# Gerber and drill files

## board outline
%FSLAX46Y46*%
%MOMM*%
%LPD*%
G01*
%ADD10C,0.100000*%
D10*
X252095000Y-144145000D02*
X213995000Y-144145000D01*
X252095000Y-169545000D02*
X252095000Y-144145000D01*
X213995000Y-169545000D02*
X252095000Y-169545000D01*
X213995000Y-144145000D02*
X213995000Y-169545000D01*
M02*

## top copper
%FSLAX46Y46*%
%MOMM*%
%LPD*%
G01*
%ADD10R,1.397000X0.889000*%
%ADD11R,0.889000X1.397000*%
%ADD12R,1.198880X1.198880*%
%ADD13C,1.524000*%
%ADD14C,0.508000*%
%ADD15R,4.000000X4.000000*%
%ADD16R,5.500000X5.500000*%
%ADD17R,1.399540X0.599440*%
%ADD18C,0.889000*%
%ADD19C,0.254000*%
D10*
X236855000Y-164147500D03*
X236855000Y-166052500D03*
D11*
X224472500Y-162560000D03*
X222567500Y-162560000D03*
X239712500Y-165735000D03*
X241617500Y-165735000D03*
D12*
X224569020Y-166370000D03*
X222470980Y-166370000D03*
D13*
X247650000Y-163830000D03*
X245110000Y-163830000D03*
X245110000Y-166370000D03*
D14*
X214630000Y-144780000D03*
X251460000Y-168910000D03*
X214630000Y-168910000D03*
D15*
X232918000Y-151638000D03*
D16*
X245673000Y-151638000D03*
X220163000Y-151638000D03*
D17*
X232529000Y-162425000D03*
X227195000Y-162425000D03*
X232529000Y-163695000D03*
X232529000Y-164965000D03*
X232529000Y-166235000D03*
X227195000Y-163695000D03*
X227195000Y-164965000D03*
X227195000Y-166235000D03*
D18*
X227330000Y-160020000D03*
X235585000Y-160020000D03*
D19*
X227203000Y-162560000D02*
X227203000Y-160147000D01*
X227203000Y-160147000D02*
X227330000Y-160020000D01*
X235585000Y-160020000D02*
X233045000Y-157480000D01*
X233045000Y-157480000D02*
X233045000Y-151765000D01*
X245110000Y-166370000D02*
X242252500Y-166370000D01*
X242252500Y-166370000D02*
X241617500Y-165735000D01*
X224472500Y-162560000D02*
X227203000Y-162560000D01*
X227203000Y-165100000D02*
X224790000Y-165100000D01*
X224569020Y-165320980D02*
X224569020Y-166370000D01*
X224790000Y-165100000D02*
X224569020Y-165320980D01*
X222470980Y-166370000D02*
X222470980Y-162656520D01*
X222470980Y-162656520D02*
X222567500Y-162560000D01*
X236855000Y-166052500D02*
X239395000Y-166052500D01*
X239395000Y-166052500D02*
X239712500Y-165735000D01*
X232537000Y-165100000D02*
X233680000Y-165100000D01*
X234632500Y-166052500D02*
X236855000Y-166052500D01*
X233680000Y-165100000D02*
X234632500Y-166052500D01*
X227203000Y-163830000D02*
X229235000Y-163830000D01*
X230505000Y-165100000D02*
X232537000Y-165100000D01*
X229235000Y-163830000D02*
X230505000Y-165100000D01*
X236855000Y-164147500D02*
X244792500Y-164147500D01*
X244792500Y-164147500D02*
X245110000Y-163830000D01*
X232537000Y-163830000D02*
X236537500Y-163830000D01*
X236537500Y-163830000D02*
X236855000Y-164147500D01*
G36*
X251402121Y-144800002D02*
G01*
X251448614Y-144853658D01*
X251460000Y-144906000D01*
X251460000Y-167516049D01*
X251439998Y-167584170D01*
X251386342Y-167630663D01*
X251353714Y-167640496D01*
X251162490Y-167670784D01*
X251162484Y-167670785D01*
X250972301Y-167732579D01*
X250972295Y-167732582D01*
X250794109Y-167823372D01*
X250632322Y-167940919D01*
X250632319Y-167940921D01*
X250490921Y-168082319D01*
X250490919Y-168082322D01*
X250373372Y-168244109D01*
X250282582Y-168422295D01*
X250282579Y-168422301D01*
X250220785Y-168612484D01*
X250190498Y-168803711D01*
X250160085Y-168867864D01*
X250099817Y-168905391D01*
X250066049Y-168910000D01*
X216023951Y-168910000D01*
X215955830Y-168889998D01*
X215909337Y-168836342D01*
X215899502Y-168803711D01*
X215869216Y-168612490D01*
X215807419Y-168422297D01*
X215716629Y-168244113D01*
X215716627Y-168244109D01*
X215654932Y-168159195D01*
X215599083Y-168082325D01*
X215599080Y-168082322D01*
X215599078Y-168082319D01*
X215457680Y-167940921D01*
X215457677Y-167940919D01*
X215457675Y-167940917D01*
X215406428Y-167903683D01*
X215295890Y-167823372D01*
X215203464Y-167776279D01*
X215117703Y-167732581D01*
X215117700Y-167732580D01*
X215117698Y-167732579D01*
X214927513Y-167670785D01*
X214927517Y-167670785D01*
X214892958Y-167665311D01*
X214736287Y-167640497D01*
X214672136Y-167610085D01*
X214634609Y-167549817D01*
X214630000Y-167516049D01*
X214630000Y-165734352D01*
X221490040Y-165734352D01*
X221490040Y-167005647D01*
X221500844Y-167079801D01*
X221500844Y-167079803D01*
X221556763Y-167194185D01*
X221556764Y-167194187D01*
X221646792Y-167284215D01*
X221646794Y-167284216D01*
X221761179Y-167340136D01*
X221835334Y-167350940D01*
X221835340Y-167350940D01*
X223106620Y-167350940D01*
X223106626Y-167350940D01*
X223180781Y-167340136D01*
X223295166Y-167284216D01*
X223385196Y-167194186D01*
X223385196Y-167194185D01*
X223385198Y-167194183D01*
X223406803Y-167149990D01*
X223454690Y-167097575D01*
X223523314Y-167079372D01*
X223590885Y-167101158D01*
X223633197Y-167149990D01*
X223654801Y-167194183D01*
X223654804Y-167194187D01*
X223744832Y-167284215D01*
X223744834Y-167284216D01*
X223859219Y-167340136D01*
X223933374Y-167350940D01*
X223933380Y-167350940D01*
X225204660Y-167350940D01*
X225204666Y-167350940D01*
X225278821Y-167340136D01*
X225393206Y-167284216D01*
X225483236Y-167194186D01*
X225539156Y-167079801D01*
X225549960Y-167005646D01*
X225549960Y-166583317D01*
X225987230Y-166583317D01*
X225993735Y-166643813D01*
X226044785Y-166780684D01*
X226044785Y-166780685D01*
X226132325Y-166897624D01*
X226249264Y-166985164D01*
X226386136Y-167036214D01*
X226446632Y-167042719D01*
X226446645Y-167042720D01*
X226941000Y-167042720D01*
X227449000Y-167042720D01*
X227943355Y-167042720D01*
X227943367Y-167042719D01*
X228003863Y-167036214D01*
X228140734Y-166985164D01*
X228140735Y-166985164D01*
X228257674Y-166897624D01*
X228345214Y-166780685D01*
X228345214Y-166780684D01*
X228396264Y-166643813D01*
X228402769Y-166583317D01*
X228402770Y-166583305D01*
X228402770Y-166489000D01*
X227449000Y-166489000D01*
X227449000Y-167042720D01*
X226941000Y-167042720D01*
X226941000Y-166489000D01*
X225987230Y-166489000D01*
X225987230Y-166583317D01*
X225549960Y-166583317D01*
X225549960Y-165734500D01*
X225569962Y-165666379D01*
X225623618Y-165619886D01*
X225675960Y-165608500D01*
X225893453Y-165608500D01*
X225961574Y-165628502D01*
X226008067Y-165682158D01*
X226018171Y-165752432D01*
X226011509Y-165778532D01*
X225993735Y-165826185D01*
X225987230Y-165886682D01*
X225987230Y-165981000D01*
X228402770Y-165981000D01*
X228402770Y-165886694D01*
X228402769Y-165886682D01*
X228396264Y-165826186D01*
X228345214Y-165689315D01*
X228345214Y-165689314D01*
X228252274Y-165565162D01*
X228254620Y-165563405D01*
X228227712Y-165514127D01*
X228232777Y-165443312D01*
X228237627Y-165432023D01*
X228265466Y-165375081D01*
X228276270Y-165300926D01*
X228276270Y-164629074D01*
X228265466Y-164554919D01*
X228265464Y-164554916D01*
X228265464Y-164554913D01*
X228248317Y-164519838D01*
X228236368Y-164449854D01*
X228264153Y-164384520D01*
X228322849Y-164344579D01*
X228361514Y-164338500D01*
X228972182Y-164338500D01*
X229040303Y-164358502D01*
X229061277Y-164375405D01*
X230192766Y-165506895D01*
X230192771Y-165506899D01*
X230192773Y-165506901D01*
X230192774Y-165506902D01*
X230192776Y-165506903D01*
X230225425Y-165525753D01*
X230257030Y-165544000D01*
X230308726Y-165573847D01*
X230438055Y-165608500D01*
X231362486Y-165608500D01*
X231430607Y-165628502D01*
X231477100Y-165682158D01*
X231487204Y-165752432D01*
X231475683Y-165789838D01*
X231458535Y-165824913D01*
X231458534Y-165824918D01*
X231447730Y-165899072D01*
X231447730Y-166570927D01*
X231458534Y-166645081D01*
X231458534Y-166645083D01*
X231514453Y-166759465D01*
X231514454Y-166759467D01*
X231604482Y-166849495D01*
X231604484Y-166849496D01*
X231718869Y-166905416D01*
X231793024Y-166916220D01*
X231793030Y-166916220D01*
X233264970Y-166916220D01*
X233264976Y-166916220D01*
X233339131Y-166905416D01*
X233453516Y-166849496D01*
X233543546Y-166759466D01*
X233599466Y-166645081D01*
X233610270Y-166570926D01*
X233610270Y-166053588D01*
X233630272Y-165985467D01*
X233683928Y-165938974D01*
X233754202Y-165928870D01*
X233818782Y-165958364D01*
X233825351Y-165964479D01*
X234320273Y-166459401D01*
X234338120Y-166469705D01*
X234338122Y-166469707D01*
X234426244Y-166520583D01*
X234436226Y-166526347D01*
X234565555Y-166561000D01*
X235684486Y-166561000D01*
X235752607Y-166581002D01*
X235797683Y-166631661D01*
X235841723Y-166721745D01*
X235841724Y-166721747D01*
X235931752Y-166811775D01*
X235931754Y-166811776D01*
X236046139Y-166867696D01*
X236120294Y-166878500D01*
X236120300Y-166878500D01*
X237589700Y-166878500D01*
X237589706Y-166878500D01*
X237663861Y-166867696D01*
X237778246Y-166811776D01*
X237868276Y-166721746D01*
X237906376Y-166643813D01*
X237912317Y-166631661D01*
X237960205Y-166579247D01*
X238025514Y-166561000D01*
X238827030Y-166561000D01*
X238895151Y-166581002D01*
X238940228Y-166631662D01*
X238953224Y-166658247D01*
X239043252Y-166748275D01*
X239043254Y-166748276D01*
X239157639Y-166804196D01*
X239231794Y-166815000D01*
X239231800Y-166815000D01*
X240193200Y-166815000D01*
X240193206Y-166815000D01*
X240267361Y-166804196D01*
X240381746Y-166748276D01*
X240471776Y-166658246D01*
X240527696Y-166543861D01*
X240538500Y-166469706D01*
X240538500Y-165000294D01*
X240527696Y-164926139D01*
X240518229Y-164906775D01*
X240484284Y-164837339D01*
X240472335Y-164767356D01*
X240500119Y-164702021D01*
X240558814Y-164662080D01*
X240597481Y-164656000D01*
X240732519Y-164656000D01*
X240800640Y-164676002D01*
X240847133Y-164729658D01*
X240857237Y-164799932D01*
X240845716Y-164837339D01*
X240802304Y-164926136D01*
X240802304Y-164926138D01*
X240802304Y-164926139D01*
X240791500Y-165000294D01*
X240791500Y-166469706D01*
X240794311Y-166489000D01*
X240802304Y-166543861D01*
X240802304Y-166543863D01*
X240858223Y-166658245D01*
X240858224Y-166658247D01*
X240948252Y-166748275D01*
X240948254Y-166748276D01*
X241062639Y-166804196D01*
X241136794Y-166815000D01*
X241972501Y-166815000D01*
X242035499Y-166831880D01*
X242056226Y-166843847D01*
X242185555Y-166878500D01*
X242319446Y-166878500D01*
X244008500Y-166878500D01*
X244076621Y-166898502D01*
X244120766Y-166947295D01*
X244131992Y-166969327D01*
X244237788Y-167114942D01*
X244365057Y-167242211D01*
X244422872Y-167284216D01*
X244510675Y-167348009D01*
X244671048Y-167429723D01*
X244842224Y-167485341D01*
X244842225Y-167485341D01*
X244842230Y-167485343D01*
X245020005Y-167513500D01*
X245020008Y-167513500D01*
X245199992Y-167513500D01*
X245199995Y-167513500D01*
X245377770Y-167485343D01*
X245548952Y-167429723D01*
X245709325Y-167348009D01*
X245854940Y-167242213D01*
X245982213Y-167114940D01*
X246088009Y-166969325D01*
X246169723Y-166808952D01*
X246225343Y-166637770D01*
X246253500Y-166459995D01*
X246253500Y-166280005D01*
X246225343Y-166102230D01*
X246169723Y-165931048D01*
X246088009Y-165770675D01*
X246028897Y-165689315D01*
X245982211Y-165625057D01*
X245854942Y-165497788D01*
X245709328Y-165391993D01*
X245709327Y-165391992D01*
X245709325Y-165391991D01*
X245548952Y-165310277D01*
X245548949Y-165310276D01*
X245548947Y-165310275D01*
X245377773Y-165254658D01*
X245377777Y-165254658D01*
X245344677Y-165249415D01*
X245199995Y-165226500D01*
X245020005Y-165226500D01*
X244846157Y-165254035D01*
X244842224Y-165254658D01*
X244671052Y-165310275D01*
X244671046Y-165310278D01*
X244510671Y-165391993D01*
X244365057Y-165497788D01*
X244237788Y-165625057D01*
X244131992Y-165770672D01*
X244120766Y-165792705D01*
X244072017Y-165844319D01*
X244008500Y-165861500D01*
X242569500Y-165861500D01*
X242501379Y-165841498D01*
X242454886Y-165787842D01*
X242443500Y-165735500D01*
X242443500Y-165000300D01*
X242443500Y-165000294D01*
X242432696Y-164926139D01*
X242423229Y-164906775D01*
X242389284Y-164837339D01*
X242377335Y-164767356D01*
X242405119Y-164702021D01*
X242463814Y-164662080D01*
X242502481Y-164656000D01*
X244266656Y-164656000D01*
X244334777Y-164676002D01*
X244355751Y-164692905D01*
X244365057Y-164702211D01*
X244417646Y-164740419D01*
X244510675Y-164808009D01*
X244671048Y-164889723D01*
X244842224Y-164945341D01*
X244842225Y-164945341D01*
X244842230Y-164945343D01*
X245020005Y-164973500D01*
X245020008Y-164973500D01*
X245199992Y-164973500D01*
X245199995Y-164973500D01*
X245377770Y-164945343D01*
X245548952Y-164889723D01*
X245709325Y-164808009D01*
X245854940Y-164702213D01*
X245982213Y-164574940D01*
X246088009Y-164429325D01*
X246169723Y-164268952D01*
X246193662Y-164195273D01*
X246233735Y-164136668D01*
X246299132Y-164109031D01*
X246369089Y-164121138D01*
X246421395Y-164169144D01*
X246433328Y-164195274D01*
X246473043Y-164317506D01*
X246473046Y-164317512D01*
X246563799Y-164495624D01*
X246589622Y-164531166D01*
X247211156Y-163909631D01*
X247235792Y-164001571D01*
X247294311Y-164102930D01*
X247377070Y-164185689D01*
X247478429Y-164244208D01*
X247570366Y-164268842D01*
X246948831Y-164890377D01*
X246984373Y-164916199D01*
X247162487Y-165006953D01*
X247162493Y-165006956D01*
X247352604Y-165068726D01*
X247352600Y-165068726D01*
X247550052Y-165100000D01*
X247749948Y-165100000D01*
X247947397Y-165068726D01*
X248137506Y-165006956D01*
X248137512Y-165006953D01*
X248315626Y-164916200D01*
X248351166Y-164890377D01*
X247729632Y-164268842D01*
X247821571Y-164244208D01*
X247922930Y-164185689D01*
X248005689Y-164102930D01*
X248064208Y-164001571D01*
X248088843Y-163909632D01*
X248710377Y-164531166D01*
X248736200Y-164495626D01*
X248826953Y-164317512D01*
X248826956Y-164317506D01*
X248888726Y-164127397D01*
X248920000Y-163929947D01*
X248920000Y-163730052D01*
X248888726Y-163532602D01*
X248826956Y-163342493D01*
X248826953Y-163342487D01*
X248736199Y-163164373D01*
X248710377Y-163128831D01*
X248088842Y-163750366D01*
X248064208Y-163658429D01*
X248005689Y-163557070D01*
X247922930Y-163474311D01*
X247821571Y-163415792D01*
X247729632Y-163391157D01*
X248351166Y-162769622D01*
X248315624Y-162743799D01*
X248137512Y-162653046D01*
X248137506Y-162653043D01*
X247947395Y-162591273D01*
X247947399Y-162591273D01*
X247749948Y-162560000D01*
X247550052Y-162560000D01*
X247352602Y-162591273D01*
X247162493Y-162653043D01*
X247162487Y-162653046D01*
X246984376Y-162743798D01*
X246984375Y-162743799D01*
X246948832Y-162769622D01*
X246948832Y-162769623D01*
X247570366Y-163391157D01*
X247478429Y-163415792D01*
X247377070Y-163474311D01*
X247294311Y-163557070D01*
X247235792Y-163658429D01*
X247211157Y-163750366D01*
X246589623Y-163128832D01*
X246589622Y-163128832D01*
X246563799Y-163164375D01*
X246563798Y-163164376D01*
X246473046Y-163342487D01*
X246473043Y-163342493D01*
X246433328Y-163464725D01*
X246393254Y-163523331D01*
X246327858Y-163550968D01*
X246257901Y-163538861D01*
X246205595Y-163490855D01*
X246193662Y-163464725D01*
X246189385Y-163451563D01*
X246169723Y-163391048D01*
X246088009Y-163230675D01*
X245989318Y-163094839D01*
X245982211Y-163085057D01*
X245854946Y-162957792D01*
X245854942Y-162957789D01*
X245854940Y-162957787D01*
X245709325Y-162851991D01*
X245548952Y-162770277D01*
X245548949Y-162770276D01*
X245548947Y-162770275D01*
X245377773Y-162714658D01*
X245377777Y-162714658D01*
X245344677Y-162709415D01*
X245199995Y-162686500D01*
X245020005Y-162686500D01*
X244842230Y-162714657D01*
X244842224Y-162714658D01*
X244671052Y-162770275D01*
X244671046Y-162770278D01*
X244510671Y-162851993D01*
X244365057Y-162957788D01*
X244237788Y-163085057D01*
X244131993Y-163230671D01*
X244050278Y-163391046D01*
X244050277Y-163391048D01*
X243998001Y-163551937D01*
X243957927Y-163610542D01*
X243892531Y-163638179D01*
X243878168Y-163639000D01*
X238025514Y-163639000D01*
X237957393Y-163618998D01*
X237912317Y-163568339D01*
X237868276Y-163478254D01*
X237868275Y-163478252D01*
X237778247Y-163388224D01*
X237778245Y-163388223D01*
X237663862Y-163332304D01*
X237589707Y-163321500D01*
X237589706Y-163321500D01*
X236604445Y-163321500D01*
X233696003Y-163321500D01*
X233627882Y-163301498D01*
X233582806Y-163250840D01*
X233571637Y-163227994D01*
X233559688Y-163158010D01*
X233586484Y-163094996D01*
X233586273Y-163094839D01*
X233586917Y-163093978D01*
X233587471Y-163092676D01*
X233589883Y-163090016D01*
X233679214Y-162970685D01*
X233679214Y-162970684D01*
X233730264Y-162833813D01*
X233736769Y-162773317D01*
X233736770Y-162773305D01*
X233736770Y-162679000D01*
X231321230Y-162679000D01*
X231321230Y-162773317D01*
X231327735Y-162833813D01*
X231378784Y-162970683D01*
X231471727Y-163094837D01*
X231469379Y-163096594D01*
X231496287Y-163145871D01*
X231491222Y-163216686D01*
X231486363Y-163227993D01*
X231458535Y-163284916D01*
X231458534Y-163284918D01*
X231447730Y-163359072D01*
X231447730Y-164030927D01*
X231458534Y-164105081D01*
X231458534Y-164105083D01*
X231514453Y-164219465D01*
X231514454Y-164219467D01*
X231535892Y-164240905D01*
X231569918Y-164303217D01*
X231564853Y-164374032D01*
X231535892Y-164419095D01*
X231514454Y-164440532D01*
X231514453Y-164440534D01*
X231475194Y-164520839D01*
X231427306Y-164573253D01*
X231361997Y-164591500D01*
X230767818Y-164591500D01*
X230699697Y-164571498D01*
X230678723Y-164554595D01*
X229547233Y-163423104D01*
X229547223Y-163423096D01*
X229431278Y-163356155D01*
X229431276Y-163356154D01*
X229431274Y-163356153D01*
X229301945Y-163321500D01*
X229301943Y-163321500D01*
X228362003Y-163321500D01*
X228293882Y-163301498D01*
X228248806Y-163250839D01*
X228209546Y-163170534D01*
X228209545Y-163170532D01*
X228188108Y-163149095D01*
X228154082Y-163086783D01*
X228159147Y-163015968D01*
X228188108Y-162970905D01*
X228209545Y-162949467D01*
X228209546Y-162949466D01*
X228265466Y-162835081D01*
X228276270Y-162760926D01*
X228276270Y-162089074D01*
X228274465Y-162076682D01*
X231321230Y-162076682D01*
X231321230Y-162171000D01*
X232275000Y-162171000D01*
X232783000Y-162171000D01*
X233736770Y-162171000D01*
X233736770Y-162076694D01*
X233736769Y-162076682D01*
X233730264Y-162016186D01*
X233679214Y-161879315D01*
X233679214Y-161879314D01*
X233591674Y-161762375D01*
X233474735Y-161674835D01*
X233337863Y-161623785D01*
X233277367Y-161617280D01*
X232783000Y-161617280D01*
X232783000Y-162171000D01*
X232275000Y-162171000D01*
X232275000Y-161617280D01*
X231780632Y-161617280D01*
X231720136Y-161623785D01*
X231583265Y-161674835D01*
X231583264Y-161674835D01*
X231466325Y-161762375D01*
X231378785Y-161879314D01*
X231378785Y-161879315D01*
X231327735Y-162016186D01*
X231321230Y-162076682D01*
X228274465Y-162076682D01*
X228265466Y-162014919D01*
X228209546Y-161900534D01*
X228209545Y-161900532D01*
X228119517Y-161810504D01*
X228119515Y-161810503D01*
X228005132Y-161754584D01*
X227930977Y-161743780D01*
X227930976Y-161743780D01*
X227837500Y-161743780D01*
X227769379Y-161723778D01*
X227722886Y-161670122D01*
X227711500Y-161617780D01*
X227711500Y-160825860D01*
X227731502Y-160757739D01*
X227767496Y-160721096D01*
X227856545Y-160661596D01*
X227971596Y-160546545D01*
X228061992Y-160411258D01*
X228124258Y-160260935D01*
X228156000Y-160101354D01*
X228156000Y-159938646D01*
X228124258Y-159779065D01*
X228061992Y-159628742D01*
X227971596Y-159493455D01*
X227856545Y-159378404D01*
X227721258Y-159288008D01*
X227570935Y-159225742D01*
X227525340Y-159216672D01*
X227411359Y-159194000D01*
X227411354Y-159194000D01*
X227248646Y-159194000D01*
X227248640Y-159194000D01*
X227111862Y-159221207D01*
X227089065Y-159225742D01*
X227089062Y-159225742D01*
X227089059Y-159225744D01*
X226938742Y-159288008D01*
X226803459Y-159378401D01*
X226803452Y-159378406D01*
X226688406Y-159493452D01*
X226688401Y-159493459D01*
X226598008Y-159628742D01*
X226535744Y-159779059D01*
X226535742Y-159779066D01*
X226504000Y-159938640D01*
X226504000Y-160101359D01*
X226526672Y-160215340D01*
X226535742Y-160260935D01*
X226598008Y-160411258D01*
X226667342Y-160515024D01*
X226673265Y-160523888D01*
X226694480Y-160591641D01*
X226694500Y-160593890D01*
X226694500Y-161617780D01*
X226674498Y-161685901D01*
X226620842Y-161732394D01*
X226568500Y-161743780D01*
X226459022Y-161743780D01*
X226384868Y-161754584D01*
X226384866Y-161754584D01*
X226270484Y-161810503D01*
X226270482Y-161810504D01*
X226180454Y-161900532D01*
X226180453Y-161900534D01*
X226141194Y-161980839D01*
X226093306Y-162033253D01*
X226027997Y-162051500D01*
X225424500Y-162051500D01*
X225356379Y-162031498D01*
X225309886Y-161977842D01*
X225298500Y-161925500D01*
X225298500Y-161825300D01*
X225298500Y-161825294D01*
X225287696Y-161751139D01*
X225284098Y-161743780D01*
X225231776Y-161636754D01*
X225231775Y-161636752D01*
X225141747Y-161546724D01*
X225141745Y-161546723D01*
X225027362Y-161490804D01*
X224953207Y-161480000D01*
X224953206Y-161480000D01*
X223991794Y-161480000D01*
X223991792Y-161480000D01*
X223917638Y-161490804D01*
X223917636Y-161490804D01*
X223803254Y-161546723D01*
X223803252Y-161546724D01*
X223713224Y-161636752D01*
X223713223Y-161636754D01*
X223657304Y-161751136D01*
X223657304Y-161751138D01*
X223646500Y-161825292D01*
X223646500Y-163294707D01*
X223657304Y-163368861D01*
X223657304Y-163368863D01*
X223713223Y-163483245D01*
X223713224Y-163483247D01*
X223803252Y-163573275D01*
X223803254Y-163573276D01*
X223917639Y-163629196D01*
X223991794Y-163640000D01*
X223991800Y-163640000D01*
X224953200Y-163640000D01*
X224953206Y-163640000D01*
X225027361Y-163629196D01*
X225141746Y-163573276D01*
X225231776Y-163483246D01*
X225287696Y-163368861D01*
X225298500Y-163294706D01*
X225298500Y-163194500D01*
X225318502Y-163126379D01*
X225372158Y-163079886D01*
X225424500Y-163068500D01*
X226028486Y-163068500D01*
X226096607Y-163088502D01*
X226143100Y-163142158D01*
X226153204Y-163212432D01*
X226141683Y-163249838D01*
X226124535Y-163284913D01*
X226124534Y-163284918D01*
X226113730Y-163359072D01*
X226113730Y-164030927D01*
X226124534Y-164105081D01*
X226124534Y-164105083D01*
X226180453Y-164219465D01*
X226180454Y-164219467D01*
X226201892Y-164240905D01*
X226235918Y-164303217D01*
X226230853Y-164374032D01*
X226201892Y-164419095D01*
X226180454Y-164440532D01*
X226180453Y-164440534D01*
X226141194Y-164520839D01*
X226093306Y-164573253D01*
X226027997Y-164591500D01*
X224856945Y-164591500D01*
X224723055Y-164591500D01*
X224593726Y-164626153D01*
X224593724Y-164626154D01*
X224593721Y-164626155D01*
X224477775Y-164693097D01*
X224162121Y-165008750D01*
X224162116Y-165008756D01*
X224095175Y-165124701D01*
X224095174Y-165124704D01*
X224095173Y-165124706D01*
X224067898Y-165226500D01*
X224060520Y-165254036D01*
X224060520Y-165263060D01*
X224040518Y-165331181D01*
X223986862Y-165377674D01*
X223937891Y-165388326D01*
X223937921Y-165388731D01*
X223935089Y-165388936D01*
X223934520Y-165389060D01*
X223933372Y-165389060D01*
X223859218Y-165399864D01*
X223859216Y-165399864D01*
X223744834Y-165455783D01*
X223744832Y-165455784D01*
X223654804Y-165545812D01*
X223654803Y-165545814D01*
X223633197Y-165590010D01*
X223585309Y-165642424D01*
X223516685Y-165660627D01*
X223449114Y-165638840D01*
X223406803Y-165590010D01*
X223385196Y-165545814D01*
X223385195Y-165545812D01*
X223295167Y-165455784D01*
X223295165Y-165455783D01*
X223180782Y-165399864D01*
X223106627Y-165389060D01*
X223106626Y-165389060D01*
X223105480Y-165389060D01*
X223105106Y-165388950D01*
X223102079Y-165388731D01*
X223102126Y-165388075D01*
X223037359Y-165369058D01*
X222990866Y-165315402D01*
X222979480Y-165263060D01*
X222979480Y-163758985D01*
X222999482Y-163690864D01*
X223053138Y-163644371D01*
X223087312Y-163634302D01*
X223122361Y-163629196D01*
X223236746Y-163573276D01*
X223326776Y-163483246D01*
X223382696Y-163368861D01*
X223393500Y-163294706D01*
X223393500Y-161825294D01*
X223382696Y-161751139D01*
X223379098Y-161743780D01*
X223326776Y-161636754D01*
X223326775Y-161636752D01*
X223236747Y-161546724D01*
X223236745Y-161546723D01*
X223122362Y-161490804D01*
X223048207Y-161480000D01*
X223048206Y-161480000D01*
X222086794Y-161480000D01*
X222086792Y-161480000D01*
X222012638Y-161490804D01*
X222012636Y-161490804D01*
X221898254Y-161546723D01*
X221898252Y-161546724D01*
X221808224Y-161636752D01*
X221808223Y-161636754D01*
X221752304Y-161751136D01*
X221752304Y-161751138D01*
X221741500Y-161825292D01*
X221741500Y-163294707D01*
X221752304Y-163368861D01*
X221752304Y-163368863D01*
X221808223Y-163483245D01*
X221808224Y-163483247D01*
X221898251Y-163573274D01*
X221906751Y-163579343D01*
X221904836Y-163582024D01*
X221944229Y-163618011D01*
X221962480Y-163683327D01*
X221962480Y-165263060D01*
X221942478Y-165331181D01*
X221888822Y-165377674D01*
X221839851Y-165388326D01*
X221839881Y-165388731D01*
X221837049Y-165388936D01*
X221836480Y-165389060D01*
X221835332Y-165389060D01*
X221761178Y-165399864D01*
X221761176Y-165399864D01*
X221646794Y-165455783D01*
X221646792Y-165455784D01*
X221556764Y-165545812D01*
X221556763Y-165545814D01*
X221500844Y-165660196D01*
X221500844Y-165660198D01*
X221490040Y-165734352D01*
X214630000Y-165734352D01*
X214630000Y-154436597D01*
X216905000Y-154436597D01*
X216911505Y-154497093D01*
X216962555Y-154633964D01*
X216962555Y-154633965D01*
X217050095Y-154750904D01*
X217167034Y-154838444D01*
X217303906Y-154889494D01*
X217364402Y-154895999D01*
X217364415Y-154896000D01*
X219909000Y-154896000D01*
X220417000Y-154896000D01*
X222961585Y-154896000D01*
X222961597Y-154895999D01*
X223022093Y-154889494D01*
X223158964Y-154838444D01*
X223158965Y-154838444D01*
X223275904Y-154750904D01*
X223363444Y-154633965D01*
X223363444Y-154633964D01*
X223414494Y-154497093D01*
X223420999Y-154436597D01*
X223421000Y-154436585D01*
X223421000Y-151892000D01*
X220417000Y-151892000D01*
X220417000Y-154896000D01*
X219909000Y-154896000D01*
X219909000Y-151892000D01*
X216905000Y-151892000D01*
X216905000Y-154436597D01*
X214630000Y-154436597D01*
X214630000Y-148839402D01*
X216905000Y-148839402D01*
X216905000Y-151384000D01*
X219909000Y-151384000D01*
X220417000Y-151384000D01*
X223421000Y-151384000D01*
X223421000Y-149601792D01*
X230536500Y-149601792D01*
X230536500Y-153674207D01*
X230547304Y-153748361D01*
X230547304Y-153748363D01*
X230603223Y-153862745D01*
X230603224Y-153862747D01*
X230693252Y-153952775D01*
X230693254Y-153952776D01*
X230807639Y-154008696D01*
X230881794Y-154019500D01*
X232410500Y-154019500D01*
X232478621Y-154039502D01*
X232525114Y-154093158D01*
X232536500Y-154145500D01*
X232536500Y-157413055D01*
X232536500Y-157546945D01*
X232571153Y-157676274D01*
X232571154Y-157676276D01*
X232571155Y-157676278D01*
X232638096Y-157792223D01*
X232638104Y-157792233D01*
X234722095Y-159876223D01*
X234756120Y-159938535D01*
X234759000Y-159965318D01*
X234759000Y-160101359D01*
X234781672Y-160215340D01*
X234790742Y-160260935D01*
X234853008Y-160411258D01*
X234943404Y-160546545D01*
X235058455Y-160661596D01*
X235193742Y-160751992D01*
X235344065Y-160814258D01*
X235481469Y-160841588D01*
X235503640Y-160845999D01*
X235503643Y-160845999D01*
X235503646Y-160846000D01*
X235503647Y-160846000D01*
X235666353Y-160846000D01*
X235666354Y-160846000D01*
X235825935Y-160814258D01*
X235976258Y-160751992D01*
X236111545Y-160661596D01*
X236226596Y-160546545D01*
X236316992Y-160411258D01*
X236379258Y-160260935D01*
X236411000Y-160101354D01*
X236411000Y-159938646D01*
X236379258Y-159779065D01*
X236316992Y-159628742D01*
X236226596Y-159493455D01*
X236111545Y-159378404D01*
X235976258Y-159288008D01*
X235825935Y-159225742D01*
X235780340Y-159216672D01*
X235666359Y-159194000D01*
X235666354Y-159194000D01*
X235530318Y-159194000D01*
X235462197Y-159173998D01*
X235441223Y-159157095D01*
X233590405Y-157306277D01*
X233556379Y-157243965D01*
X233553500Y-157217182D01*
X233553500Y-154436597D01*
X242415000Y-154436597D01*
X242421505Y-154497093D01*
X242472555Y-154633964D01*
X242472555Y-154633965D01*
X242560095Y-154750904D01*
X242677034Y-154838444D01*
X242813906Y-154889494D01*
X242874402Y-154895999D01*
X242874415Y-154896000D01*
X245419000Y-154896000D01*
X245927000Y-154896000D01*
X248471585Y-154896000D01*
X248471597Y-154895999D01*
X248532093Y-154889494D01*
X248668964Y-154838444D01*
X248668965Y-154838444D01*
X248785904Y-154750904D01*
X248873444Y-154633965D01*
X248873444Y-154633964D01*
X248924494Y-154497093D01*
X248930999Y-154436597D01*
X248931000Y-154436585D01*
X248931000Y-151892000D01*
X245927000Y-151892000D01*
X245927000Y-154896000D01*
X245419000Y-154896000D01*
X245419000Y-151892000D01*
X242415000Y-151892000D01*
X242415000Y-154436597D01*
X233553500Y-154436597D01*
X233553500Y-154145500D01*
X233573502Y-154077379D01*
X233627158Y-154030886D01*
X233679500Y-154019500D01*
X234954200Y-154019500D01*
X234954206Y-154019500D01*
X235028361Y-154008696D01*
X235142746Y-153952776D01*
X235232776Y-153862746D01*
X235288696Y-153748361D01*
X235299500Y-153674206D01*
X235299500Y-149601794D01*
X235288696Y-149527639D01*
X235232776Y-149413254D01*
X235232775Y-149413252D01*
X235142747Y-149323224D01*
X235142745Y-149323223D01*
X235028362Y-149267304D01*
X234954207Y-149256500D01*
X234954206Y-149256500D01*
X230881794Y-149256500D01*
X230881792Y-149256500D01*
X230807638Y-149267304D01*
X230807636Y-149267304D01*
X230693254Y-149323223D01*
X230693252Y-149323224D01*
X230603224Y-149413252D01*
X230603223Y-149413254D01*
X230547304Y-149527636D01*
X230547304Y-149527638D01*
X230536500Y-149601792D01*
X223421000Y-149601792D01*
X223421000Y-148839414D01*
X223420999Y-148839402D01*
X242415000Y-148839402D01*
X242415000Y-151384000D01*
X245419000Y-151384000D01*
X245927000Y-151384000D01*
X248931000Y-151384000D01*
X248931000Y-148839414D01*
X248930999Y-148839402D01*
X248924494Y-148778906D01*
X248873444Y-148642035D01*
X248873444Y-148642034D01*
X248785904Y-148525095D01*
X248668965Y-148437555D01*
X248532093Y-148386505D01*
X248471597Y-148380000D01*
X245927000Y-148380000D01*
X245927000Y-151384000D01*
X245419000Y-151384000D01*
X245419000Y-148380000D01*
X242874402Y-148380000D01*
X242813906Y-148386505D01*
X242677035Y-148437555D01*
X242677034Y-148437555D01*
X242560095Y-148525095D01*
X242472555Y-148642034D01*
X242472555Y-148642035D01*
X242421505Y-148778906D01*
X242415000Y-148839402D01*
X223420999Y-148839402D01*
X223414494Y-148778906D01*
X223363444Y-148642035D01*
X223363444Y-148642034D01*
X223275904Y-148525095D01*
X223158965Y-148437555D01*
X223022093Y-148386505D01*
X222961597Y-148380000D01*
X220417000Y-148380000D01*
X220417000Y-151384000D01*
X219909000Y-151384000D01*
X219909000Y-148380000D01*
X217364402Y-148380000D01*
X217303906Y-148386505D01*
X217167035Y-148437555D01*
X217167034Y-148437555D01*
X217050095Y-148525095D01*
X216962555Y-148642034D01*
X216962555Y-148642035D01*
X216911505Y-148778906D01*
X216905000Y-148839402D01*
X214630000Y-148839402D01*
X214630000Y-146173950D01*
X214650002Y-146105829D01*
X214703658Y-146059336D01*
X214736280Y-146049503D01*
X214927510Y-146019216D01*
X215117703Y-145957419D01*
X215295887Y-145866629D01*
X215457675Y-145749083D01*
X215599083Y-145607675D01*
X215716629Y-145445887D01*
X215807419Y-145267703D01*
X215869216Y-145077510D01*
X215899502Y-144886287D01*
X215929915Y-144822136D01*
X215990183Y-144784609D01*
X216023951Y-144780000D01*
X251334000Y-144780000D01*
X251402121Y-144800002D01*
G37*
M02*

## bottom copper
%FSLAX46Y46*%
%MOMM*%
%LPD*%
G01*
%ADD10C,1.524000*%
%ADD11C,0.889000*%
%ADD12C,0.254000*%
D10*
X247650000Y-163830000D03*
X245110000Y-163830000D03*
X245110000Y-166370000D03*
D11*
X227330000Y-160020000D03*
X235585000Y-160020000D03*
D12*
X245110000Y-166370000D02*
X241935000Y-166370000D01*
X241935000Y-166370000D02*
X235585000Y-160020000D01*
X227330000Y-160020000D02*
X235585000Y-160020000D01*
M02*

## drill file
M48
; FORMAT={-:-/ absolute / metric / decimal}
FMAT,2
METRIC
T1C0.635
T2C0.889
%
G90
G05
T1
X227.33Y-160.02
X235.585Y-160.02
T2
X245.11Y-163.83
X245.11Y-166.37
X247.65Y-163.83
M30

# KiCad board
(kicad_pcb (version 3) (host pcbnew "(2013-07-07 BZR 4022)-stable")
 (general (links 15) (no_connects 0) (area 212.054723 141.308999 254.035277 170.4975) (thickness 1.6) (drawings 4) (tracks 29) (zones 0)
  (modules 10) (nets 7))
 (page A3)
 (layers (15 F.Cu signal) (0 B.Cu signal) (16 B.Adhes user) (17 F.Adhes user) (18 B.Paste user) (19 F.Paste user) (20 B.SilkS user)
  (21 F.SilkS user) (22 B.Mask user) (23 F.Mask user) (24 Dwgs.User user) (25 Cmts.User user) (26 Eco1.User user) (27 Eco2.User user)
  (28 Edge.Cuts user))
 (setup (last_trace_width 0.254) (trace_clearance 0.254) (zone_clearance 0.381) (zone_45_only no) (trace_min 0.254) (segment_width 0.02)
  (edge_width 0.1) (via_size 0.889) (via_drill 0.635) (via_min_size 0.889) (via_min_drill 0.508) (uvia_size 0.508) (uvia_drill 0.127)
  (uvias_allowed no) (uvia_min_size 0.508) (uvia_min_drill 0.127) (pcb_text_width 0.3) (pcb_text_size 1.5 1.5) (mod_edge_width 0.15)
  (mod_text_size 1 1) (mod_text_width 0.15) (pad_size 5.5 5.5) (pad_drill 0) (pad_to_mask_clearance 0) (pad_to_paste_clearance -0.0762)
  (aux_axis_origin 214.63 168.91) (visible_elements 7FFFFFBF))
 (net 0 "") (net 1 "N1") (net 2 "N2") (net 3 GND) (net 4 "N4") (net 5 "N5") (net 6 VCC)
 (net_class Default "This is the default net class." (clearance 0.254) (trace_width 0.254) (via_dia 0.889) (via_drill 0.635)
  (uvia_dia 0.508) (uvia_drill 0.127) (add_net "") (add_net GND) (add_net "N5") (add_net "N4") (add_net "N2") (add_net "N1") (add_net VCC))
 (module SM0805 (layer F.Cu) (at 236.855 165.1 270)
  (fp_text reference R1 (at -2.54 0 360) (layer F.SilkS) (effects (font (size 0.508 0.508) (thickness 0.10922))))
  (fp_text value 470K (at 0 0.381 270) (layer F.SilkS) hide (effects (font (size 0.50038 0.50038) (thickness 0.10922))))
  (pad 1 smd rect (at -0.9525 0 270) (size 0.889 1.397) (layers F.Cu F.Paste F.Mask) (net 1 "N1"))
  (pad 2 smd rect (at 0.9525 0 270) (size 0.889 1.397) (layers F.Cu F.Paste F.Mask) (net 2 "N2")))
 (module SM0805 (layer F.Cu) (at 223.52 162.56 180)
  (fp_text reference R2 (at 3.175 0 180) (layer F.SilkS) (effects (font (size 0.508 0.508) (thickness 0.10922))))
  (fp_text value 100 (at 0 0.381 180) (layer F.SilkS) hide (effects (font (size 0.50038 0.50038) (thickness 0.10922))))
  (pad 1 smd rect (at -0.9525 0 180) (size 0.889 1.397) (layers F.Cu F.Paste F.Mask) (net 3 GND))
  (pad 2 smd rect (at 0.9525 0 180) (size 0.889 1.397) (layers F.Cu F.Paste F.Mask) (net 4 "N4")))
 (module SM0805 (layer F.Cu) (at 240.665 165.735)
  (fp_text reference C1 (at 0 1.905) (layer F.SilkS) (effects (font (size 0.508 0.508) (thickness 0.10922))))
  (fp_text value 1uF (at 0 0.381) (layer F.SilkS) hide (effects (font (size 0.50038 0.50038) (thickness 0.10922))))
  (pad 1 smd rect (at -0.9525 0) (size 0.889 1.397) (layers F.Cu F.Paste F.Mask) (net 2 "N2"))
  (pad 2 smd rect (at 0.9525 0) (size 0.889 1.397) (layers F.Cu F.Paste F.Mask) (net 3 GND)))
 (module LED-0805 (layer F.Cu) (at 223.52 166.37 180)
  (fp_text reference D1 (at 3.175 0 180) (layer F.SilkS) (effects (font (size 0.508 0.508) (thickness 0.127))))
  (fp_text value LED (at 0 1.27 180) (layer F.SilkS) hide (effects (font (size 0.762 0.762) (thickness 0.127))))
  (pad 1 smd rect (at -1.04902 0 180) (size 1.19888 1.19888) (layers F.Cu F.Paste F.Mask) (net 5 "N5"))
  (pad 2 smd rect (at 1.04902 0 180) (size 1.19888 1.19888) (layers F.Cu F.Paste F.Mask) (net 4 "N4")))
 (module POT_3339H (layer F.Cu) (at 245.11 163.83 180)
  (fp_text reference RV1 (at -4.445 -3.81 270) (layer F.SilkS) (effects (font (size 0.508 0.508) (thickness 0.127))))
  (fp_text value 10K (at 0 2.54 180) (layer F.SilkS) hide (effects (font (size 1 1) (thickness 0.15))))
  (pad 1 thru_hole circle (at -2.54 0 180) (size 1.524 1.524) (drill 0.889) (layers *.Cu *.Mask F.SilkS) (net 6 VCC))
  (pad 2 thru_hole circle (at 0 0 180) (size 1.524 1.524) (drill 0.889) (layers *.Cu *.Mask F.SilkS) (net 1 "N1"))
  (pad 3 thru_hole circle (at 0 -2.54 180) (size 1.524 1.524) (drill 0.889) (layers *.Cu *.Mask F.SilkS) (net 3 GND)))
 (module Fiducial (layer F.Cu) (at 214.63 144.78)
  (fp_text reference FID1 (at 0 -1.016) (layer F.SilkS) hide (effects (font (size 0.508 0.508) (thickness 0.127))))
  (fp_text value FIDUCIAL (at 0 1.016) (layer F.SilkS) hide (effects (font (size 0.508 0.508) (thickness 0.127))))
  (pad "" smd circle (at 0 0) (size 0.508 0.508) (layers F.Cu F.Mask) (solder_mask_margin 1.016) (clearance 1.016) (zone_connect 1)
   (thermal_width 1)))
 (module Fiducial (layer F.Cu) (at 251.46 168.91)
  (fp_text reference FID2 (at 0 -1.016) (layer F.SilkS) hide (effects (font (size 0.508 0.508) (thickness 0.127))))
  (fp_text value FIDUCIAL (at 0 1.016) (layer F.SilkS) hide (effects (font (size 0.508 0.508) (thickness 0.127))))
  (pad "" smd circle (at 0 0) (size 0.508 0.508) (layers F.Cu F.Mask) (solder_mask_margin 1.016) (clearance 1.016) (zone_connect 1)
   (thermal_width 1)))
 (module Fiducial (layer F.Cu) (at 214.63 168.91)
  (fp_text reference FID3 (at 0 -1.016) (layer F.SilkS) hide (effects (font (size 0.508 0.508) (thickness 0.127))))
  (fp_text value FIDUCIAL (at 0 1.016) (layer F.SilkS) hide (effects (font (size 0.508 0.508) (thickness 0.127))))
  (pad "" smd circle (at 0 0) (size 0.508 0.508) (layers F.Cu F.Mask) (solder_mask_margin 1.016) (clearance 1.016) (zone_connect 1)
   (thermal_width 1)))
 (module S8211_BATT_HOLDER (layer F.Cu) (at 232.918 151.638 90)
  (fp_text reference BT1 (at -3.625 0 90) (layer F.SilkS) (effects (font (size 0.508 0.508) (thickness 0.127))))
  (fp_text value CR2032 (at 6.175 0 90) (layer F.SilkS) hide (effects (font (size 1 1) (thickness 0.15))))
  (pad 2 smd rect (at 0 0 180) (size 4 4) (layers F.Cu F.Mask) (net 3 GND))
  (pad 1 smd rect (at 0 12.755 180) (size 5.5 5.5) (layers F.Cu F.Paste F.Mask) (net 6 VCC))
  (pad 1 smd rect (at 0 -12.755 180) (size 5.5 5.5) (layers F.Cu F.Paste F.Mask) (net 6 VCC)))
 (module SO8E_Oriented (layer F.Cu) (at 229.87 164.338)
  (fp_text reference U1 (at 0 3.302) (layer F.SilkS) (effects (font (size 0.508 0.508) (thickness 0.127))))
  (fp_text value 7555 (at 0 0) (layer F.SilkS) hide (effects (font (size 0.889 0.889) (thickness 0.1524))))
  (pad 8 smd rect (at 2.659 -1.913 270) (size 0.59944 1.39954) (layers F.Cu F.Paste F.Mask) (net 6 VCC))
  (pad 1 smd rect (at -2.675 -1.913 270) (size 0.59944 1.39954) (layers F.Cu F.Paste F.Mask) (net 3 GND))
  (pad 7 smd rect (at 2.659 -0.643 270) (size 0.59944 1.39954) (layers F.Cu F.Paste F.Mask) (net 1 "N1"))
  (pad 6 smd rect (at 2.659 0.627 270) (size 0.59944 1.39954) (layers F.Cu F.Paste F.Mask) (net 2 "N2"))
  (pad 5 smd rect (at 2.659 1.897 270) (size 0.59944 1.39954) (layers F.Cu F.Paste F.Mask))
  (pad 2 smd rect (at -2.675 -0.643 270) (size 0.59944 1.39954) (layers F.Cu F.Paste F.Mask) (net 2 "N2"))
  (pad 3 smd rect (at -2.675 0.627 270) (size 0.59944 1.39954) (layers F.Cu F.Paste F.Mask) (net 5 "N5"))
  (pad 4 smd rect (at -2.675 1.897 270) (size 0.59944 1.39954) (layers F.Cu F.Paste F.Mask) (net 6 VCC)))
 (gr_line (start 252.095 144.145) (end 213.995 144.145) (angle 90) (layer Edge.Cuts) (width 0.1))
 (gr_line (start 252.095 169.545) (end 252.095 144.145) (angle 90) (layer Edge.Cuts) (width 0.1))
 (gr_line (start 213.995 169.545) (end 252.095 169.545) (angle 90) (layer Edge.Cuts) (width 0.1))
 (gr_line (start 213.995 144.145) (end 213.995 169.545) (angle 90) (layer Edge.Cuts) (width 0.1))
 (segment (start 245.11 166.37) (end 241.935 166.37) (width 0.254) (layer B.Cu) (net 3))
 (segment (start 241.935 166.37) (end 235.585 160.02) (width 0.254) (layer B.Cu) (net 3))
 (segment (start 227.203 162.56) (end 227.203 160.147) (width 0.254) (layer F.Cu) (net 3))
 (segment (start 227.203 160.147) (end 227.33 160.02) (width 0.254) (layer F.Cu) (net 3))
 (via (at 227.33 160.02) (size 0.889) (layers F.Cu B.Cu) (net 3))
 (segment (start 227.33 160.02) (end 235.585 160.02) (width 0.254) (layer B.Cu) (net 3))
 (via (at 235.585 160.02) (size 0.889) (layers F.Cu B.Cu) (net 3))
 (segment (start 235.585 160.02) (end 233.045 157.48) (width 0.254) (layer F.Cu) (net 3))
 (segment (start 233.045 157.48) (end 233.045 151.765) (width 0.254) (layer F.Cu) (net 3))
 (segment (start 245.11 166.37) (end 242.2525 166.37) (width 0.254) (layer F.Cu) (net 3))
 (segment (start 242.2525 166.37) (end 241.6175 165.735) (width 0.254) (layer F.Cu) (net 3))
 (segment (start 224.4725 162.56) (end 227.203 162.56) (width 0.254) (layer F.Cu) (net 3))
 (segment (start 227.203 165.1) (end 224.79 165.1) (width 0.254) (layer F.Cu) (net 5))
 (segment (start 224.56902 165.32098) (end 224.56902 166.37) (width 0.254) (layer F.Cu) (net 5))
 (segment (start 224.79 165.1) (end 224.56902 165.32098) (width 0.254) (layer F.Cu) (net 5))
 (segment (start 222.47098 166.37) (end 222.47098 162.65652) (width 0.254) (layer F.Cu) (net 4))
 (segment (start 222.47098 162.65652) (end 222.5675 162.56) (width 0.254) (layer F.Cu) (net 4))
 (segment (start 236.855 166.0525) (end 239.395 166.0525) (width 0.254) (layer F.Cu) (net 2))
 (segment (start 239.395 166.0525) (end 239.7125 165.735) (width 0.254) (layer F.Cu) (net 2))
 (segment (start 232.537 165.1) (end 233.68 165.1) (width 0.254) (layer F.Cu) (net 2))
 (segment (start 234.6325 166.0525) (end 236.855 166.0525) (width 0.254) (layer F.Cu) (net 2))
 (segment (start 233.68 165.1) (end 234.6325 166.0525) (width 0.254) (layer F.Cu) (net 2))
 (segment (start 227.203 163.83) (end 229.235 163.83) (width 0.254) (layer F.Cu) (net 2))
 (segment (start 230.505 165.1) (end 232.537 165.1) (width 0.254) (layer F.Cu) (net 2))
 (segment (start 229.235 163.83) (end 230.505 165.1) (width 0.254) (layer F.Cu) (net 2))
 (segment (start 236.855 164.1475) (end 244.7925 164.1475) (width 0.254) (layer F.Cu) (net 1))
 (segment (start 244.7925 164.1475) (end 245.11 163.83) (width 0.254) (layer F.Cu) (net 1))
 (segment (start 232.537 163.83) (end 236.5375 163.83) (width 0.254) (layer F.Cu) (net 1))
 (segment (start 236.5375 163.83) (end 236.855 164.1475) (width 0.254) (layer F.Cu) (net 1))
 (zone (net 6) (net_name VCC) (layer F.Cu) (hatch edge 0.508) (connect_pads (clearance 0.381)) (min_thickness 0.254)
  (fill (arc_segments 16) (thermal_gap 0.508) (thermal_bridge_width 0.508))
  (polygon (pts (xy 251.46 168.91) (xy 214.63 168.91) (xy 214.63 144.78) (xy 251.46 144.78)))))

